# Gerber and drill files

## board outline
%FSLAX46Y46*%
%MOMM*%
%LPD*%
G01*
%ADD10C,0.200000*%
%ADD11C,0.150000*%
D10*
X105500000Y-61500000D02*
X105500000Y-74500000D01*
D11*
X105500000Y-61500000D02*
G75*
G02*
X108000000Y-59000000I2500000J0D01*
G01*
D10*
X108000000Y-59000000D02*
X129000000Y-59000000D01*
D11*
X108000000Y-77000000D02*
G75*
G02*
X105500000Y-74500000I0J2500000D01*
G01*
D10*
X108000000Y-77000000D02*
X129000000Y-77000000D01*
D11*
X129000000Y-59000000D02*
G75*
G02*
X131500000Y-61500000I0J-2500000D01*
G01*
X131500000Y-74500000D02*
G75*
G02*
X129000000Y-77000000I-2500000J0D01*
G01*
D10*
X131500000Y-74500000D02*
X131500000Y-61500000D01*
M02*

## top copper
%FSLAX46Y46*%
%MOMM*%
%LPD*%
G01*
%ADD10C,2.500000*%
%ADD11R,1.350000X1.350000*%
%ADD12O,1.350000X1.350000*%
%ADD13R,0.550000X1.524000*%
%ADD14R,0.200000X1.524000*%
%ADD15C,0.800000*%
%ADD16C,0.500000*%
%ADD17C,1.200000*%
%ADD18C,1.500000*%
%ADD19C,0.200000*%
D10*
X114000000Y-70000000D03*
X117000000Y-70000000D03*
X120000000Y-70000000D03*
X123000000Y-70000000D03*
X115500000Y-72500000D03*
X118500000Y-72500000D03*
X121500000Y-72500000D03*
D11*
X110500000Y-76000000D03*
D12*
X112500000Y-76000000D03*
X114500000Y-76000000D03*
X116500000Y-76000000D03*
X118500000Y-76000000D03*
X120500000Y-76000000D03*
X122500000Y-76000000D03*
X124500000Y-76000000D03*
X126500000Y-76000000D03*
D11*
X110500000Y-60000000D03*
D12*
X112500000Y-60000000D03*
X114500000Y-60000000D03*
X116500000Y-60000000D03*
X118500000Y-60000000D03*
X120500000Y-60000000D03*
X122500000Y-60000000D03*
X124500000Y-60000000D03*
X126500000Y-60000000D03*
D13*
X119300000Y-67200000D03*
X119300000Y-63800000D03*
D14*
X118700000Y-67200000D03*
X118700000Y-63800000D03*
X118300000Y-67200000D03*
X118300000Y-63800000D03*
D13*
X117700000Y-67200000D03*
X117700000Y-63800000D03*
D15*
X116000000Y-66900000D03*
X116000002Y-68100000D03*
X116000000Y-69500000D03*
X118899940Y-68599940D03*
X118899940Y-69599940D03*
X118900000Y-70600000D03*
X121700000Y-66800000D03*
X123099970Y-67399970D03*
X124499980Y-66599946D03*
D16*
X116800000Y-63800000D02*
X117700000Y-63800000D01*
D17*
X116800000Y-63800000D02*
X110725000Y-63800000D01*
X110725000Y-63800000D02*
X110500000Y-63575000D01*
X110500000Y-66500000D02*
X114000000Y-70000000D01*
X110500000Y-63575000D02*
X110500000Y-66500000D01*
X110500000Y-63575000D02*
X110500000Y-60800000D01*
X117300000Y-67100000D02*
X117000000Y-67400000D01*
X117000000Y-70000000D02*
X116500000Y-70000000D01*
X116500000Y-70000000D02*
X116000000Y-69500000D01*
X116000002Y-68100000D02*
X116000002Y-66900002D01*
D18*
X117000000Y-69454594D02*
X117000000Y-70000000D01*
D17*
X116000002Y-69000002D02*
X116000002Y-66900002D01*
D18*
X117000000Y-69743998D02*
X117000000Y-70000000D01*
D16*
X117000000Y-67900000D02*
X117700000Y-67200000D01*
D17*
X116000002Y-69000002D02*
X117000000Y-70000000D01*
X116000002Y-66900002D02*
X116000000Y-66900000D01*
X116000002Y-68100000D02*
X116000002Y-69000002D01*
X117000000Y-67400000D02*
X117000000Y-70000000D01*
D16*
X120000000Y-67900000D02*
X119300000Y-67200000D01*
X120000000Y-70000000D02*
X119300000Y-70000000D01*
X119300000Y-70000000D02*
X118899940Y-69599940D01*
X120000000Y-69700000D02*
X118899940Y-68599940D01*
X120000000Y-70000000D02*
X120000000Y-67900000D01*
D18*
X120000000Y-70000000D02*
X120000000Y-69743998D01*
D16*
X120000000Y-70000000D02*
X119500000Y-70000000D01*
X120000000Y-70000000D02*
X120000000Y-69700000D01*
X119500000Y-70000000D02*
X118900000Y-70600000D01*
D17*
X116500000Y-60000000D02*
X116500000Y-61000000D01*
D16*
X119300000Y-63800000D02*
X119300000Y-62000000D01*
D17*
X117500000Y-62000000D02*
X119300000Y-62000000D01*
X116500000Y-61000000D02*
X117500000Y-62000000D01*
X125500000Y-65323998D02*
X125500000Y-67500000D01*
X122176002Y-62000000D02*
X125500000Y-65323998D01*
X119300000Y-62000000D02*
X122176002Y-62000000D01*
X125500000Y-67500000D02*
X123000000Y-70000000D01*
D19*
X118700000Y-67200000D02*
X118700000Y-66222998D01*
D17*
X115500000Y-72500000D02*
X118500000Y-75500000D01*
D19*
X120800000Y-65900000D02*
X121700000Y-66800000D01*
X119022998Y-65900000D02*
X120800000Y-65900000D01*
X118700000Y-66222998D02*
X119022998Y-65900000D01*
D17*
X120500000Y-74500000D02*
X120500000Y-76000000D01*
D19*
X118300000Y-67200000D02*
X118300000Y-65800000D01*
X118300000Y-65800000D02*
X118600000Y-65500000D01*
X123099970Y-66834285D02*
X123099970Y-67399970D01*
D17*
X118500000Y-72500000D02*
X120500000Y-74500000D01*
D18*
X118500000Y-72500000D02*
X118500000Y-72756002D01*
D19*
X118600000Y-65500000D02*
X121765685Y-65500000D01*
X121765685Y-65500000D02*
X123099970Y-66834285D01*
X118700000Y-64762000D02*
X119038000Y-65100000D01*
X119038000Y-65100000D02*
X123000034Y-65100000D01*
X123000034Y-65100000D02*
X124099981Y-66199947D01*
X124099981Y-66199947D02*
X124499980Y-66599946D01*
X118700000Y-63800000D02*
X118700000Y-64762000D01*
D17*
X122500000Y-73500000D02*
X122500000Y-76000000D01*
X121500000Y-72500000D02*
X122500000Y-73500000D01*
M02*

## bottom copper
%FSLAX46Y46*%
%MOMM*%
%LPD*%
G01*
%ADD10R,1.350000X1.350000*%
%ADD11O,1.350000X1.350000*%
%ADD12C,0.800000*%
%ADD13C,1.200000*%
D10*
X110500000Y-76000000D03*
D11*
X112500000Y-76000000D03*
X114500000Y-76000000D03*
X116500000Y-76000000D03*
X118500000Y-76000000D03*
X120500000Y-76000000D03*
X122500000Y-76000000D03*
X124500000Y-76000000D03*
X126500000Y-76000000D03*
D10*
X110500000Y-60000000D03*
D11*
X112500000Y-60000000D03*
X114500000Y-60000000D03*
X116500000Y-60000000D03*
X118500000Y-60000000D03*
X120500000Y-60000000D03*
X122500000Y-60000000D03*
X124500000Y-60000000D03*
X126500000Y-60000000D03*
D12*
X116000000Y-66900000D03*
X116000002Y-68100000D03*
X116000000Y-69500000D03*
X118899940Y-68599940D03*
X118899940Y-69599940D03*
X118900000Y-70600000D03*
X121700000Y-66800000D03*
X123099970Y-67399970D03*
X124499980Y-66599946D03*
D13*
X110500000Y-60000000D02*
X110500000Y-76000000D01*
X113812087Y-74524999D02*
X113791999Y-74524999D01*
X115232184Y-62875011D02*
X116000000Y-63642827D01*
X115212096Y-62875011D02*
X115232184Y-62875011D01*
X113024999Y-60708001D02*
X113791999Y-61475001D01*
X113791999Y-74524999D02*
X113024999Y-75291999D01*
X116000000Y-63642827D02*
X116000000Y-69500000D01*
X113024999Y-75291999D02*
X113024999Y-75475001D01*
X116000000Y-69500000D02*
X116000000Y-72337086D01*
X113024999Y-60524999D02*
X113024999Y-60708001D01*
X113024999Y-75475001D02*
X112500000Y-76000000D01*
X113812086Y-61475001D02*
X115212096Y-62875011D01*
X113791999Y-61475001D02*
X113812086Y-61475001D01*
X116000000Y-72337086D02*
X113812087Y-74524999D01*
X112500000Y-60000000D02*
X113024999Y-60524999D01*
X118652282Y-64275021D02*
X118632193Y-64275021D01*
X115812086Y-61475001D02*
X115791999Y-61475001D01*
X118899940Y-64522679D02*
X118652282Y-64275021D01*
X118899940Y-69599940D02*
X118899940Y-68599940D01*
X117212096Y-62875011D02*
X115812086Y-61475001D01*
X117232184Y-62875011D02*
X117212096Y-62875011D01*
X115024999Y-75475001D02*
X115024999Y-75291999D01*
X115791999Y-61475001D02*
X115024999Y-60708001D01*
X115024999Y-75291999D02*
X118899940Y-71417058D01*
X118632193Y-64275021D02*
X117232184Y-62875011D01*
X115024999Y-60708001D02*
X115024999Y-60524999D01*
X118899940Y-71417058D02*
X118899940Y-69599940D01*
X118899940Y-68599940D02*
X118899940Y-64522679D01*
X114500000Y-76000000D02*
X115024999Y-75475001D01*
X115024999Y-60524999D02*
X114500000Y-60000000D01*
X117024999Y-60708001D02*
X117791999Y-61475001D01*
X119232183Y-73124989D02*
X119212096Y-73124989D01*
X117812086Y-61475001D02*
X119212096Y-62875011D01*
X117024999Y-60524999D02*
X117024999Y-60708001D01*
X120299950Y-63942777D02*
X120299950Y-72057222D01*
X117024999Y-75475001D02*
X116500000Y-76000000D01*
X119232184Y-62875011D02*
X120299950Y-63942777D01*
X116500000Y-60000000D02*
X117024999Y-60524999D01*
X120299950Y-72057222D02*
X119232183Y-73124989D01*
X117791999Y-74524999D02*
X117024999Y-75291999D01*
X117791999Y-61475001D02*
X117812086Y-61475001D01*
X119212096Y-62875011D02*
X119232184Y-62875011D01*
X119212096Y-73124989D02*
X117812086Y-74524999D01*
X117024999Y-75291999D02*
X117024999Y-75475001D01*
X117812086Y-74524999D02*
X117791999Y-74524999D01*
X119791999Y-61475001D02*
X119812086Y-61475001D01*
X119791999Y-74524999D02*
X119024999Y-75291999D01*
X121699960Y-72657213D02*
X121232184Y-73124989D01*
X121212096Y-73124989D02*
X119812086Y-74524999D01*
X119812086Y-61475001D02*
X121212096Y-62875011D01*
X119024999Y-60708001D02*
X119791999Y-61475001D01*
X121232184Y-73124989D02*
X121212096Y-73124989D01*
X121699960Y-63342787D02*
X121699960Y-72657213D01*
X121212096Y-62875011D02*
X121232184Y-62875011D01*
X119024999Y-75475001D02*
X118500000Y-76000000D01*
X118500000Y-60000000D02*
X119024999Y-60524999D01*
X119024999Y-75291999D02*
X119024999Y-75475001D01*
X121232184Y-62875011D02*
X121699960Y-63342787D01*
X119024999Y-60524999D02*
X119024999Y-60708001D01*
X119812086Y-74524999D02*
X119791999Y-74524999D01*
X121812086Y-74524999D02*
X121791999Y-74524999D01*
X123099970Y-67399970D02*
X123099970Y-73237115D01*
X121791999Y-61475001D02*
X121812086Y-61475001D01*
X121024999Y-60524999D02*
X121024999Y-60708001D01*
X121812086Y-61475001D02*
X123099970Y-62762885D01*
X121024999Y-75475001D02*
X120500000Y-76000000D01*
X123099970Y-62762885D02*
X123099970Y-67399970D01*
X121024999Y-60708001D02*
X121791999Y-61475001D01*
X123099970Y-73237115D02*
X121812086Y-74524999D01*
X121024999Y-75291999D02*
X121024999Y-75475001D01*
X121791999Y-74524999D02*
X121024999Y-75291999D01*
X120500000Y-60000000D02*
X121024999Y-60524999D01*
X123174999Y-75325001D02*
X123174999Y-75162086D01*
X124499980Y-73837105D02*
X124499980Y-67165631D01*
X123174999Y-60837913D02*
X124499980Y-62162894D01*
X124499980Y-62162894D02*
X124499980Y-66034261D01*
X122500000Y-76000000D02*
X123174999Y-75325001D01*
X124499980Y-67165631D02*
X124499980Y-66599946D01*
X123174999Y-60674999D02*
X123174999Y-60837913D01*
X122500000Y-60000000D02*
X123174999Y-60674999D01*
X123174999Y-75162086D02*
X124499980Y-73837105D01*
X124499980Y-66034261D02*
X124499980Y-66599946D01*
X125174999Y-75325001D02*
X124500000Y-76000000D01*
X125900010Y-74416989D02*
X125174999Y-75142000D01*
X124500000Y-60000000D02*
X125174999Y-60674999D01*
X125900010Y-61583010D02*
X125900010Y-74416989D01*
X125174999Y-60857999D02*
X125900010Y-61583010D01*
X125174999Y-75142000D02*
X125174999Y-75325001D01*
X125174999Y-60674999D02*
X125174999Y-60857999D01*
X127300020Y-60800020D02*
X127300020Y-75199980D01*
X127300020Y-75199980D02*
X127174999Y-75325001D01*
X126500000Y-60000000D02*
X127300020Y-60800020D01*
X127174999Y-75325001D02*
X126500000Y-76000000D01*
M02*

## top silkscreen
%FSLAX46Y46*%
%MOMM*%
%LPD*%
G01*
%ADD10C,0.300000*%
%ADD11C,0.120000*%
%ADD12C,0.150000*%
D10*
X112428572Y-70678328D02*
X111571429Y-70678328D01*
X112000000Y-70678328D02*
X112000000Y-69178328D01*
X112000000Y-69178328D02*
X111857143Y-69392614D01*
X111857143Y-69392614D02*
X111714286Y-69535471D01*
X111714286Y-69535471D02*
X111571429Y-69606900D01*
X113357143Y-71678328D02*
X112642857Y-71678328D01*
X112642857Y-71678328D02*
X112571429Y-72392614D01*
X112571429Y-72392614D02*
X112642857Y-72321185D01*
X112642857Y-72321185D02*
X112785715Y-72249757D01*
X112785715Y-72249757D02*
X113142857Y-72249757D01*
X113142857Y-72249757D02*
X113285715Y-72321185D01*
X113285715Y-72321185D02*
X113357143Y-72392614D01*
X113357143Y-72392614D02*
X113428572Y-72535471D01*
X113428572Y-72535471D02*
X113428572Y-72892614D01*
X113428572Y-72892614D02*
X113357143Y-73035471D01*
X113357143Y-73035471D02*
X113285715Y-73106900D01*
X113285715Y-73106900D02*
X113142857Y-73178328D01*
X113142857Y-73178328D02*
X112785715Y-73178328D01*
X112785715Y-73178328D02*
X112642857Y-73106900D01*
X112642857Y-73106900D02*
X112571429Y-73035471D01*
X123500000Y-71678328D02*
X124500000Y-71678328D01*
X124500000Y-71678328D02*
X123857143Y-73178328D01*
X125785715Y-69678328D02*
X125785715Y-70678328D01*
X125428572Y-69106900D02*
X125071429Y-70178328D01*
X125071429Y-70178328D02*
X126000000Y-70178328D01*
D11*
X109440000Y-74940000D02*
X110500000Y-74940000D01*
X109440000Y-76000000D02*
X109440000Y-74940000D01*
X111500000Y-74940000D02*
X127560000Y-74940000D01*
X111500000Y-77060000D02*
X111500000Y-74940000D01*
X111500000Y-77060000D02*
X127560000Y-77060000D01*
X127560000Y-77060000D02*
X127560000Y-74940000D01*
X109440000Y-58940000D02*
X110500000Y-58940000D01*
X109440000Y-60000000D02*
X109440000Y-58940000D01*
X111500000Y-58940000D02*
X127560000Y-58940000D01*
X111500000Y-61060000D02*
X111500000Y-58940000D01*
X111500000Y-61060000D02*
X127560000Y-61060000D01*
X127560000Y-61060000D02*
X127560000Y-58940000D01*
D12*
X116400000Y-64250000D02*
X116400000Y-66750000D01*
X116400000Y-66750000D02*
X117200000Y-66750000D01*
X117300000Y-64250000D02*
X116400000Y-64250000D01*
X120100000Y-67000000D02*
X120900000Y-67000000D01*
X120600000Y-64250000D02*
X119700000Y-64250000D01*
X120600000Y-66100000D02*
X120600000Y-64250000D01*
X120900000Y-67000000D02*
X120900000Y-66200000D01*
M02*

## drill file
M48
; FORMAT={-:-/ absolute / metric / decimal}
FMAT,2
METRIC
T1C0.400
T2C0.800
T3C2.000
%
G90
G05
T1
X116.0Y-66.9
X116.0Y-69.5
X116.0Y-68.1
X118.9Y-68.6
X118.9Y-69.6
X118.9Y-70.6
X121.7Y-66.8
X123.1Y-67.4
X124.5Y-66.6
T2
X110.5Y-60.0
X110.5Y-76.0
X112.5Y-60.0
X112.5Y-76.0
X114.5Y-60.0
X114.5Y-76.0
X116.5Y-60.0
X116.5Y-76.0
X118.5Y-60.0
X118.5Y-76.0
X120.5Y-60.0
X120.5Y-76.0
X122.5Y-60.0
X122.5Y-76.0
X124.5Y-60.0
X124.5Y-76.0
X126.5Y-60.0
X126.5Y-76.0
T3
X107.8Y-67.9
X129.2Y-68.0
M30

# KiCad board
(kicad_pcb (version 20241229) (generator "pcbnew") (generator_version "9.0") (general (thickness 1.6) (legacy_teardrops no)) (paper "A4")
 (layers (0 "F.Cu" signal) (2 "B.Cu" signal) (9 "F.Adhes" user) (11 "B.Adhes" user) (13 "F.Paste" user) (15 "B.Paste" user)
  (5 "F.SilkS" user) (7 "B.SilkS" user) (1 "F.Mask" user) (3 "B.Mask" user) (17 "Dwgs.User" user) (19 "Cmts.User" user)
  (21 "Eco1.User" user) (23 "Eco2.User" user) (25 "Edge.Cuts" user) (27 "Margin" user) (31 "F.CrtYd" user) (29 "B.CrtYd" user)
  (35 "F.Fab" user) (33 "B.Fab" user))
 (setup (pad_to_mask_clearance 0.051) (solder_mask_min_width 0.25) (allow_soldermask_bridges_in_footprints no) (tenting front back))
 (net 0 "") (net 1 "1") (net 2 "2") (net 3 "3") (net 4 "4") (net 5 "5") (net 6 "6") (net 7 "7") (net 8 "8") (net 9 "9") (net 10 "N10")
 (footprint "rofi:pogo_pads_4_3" (layer "F.Cu") (at 118.5 70)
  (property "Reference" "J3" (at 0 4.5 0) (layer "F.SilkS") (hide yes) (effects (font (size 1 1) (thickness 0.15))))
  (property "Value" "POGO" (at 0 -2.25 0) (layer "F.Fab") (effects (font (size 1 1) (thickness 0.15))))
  (pad "1" smd circle (at -4.5 0) (size 2.5 2.5) (layers "F.Cu" "F.Mask" "F.Paste") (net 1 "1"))
  (pad "2" smd circle (at -1.5 0) (size 2.5 2.5) (layers "F.Cu" "F.Mask" "F.Paste") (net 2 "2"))
  (pad "3" smd circle (at 1.5 0) (size 2.5 2.5) (layers "F.Cu" "F.Mask" "F.Paste") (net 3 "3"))
  (pad "4" smd circle (at 4.5 0) (size 2.5 2.5) (layers "F.Cu" "F.Mask" "F.Paste") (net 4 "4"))
  (pad "5" smd circle (at -3 2.5) (size 2.5 2.5) (layers "F.Cu" "F.Mask" "F.Paste") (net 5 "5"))
  (pad "6" smd circle (at 0 2.5) (size 2.5 2.5) (layers "F.Cu" "F.Mask" "F.Paste") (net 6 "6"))
  (pad "7" smd circle (at 3 2.5) (size 2.5 2.5) (layers "F.Cu" "F.Mask" "F.Paste") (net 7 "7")))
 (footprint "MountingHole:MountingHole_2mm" (layer "F.Cu") (at 129.2 68)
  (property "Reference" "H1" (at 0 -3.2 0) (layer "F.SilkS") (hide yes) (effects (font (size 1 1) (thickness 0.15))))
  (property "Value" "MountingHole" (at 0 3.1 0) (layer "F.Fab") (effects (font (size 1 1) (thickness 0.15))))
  (pad "" np_thru_hole circle (at 0 0) (size 2 2) (drill 2) (layers "*.Cu" "*.Mask")))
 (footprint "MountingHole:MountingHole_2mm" (layer "F.Cu") (at 107.8 67.9)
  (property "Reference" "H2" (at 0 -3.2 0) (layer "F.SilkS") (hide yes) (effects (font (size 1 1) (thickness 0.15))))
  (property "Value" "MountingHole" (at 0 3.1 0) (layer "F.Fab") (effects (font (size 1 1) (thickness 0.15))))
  (pad "" np_thru_hole circle (at 0 0) (size 2 2) (drill 2) (layers "*.Cu" "*.Mask")))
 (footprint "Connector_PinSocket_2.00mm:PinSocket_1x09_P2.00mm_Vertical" (layer "F.Cu") (at 110.5 76 90)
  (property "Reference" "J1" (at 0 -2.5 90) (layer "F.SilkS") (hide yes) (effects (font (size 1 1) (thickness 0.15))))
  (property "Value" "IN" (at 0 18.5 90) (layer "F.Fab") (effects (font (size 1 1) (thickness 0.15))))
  (fp_line (start 1.06 -1.06) (end 1.06 0) (stroke (width 0.12) (type solid)) (layer "F.SilkS"))
  (fp_line (start 0 -1.06) (end 1.06 -1.06) (stroke (width 0.12) (type solid)) (layer "F.SilkS"))
  (fp_line (start 1.06 1) (end 1.06 17.06) (stroke (width 0.12) (type solid)) (layer "F.SilkS"))
  (fp_line (start -1.06 1) (end 1.06 1) (stroke (width 0.12) (type solid)) (layer "F.SilkS"))
  (fp_line (start -1.06 1) (end -1.06 17.06) (stroke (width 0.12) (type solid)) (layer "F.SilkS"))
  (fp_line (start -1.06 17.06) (end 1.06 17.06) (stroke (width 0.12) (type solid)) (layer "F.SilkS"))
  (pad "1" thru_hole rect (at 0 0 90) (size 1.35 1.35) (drill 0.8) (layers "*.Cu" "*.Mask") (remove_unused_layers no) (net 1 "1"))
  (pad "2" thru_hole oval (at 0 2 90) (size 1.35 1.35) (drill 0.8) (layers "*.Cu" "*.Mask") (remove_unused_layers no) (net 2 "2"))
  (pad "3" thru_hole oval (at 0 4 90) (size 1.35 1.35) (drill 0.8) (layers "*.Cu" "*.Mask") (remove_unused_layers no) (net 3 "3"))
  (pad "4" thru_hole oval (at 0 6 90) (size 1.35 1.35) (drill 0.8) (layers "*.Cu" "*.Mask") (remove_unused_layers no) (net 4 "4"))
  (pad "5" thru_hole oval (at 0 8 90) (size 1.35 1.35) (drill 0.8) (layers "*.Cu" "*.Mask") (remove_unused_layers no) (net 5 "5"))
  (pad "6" thru_hole oval (at 0 10 90) (size 1.35 1.35) (drill 0.8) (layers "*.Cu" "*.Mask") (remove_unused_layers no) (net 6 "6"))
  (pad "7" thru_hole oval (at 0 12 90) (size 1.35 1.35) (drill 0.8) (layers "*.Cu" "*.Mask") (remove_unused_layers no) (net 7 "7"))
  (pad "8" thru_hole oval (at 0 14 90) (size 1.35 1.35) (drill 0.8) (layers "*.Cu" "*.Mask") (remove_unused_layers no) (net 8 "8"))
  (pad "9" thru_hole oval (at 0 16 90) (size 1.35 1.35) (drill 0.8) (layers "*.Cu" "*.Mask") (remove_unused_layers no) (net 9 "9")))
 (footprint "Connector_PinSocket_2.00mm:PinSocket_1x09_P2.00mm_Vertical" (layer "F.Cu") (at 110.5 60 90)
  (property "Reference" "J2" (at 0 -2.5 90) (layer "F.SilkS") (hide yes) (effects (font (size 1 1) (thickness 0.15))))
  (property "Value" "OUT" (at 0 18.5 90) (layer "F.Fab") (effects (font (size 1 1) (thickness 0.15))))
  (fp_line (start 1.06 -1.06) (end 1.06 0) (stroke (width 0.12) (type solid)) (layer "F.SilkS"))
  (fp_line (start 0 -1.06) (end 1.06 -1.06) (stroke (width 0.12) (type solid)) (layer "F.SilkS"))
  (fp_line (start 1.06 1) (end 1.06 17.06) (stroke (width 0.12) (type solid)) (layer "F.SilkS"))
  (fp_line (start -1.06 1) (end 1.06 1) (stroke (width 0.12) (type solid)) (layer "F.SilkS"))
  (fp_line (start -1.06 1) (end -1.06 17.06) (stroke (width 0.12) (type solid)) (layer "F.SilkS"))
  (fp_line (start -1.06 17.06) (end 1.06 17.06) (stroke (width 0.12) (type solid)) (layer "F.SilkS"))
  (pad "1" thru_hole rect (at 0 0 90) (size 1.35 1.35) (drill 0.8) (layers "*.Cu" "*.Mask") (remove_unused_layers no) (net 1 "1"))
  (pad "2" thru_hole oval (at 0 2 90) (size 1.35 1.35) (drill 0.8) (layers "*.Cu" "*.Mask") (remove_unused_layers no) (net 2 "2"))
  (pad "3" thru_hole oval (at 0 4 90) (size 1.35 1.35) (drill 0.8) (layers "*.Cu" "*.Mask") (remove_unused_layers no) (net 3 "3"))
  (pad "4" thru_hole oval (at 0 6 90) (size 1.35 1.35) (drill 0.8) (layers "*.Cu" "*.Mask") (remove_unused_layers no) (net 4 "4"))
  (pad "5" thru_hole oval (at 0 8 90) (size 1.35 1.35) (drill 0.8) (layers "*.Cu" "*.Mask") (remove_unused_layers no) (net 5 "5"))
  (pad "6" thru_hole oval (at 0 10 90) (size 1.35 1.35) (drill 0.8) (layers "*.Cu" "*.Mask") (remove_unused_layers no) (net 6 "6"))
  (pad "7" thru_hole oval (at 0 12 90) (size 1.35 1.35) (drill 0.8) (layers "*.Cu" "*.Mask") (remove_unused_layers no) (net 7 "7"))
  (pad "8" thru_hole oval (at 0 14 90) (size 1.35 1.35) (drill 0.8) (layers "*.Cu" "*.Mask") (remove_unused_layers no) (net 8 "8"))
  (pad "9" thru_hole oval (at 0 16 90) (size 1.35 1.35) (drill 0.8) (layers "*.Cu" "*.Mask") (remove_unused_layers no) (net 9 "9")))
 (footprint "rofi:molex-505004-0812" (layer "F.Cu") (at 118.5 65.5 180)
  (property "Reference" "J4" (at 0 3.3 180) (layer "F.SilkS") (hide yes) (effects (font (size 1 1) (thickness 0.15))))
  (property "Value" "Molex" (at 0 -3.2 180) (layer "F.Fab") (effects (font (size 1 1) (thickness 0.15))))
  (fp_line (start 2.1 1.25) (end 2.1 -1.25) (stroke (width 0.15) (type solid)) (layer "F.SilkS"))
  (fp_line (start 2.1 -1.25) (end 1.3 -1.25) (stroke (width 0.15) (type solid)) (layer "F.SilkS"))
  (fp_line (start 1.2 1.25) (end 2.1 1.25) (stroke (width 0.15) (type solid)) (layer "F.SilkS"))
  (fp_line (start -1.6 -1.5) (end -2.4 -1.5) (stroke (width 0.15) (type solid)) (layer "F.SilkS"))
  (fp_line (start -2.1 1.25) (end -1.2 1.25) (stroke (width 0.15) (type solid)) (layer "F.SilkS"))
  (fp_line (start -2.1 -0.6) (end -2.1 1.25) (stroke (width 0.15) (type solid)) (layer "F.SilkS"))
  (fp_line (start -2.4 -1.5) (end -2.4 -0.7) (stroke (width 0.15) (type solid)) (layer "F.SilkS"))
  (pad "1" smd rect (at -0.8 -1.7 180) (size 0.55 1.524) (layers "F.Cu" "F.Mask" "F.Paste") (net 3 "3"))
  (pad "2" smd rect (at -0.8 1.7 180) (size 0.55 1.524) (layers "F.Cu" "F.Mask" "F.Paste") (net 4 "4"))
  (pad "3" smd rect (at -0.2 -1.7 180) (size 0.2 1.524) (layers "F.Cu" "F.Mask" "F.Paste") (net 5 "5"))
  (pad "4" smd rect (at -0.2 1.7 180) (size 0.2 1.524) (layers "F.Cu" "F.Mask" "F.Paste") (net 7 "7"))
  (pad "5" smd rect (at 0.2 -1.7 180) (size 0.2 1.524) (layers "F.Cu" "F.Mask" "F.Paste") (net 6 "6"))
  (pad "6" smd rect (at 0.2 1.7 180) (size 0.2 1.524) (layers "F.Cu" "F.Mask" "F.Paste") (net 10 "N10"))
  (pad "7" smd rect (at 0.8 -1.7 180) (size 0.55 1.524) (layers "F.Cu" "F.Mask" "F.Paste") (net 2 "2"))
  (pad "8" smd rect (at 0.8 1.7 180) (size 0.55 1.524) (layers "F.Cu" "F.Mask" "F.Paste") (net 1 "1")))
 (gr_line (start 105.5 61.5) (end 105.5 74.5) (stroke (width 0.2) (type solid)) (layer "Edge.Cuts"))
 (gr_arc (start 105.5 61.5) (mid 106.232233 59.732233) (end 108 59) (stroke (width 0.15) (type solid)) (layer "Edge.Cuts"))
 (gr_line (start 108 59) (end 129 59) (stroke (width 0.2) (type solid)) (layer "Edge.Cuts"))
 (gr_arc (start 108 77) (mid 106.232233 76.267767) (end 105.5 74.5) (stroke (width 0.15) (type solid)) (layer "Edge.Cuts"))
 (gr_line (start 108 77) (end 129 77) (stroke (width 0.2) (type solid)) (layer "Edge.Cuts"))
 (gr_arc (start 129 59) (mid 130.767767 59.732233) (end 131.5 61.5) (stroke (width 0.15) (type solid)) (layer "Edge.Cuts"))
 (gr_arc (start 131.5 74.5) (mid 130.767767 76.267767) (end 129 77) (stroke (width 0.15) (type solid)) (layer "Edge.Cuts"))
 (gr_line (start 131.5 74.5) (end 131.5 61.5) (stroke (width 0.2) (type solid)) (layer "Edge.Cuts"))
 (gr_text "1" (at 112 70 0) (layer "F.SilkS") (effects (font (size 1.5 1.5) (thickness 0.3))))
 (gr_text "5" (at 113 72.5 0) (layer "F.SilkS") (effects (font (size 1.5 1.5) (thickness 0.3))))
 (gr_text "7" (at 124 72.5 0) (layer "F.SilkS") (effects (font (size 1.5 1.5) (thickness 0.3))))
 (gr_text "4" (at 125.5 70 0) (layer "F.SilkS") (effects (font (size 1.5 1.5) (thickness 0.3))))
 (segment (start 116.8 63.8) (end 117.7 63.8) (width 0.5) (layer "F.Cu") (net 1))
 (segment (start 116.8 63.8) (end 110.725 63.8) (width 1.2) (layer "F.Cu") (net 1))
 (segment (start 110.725 63.8) (end 110.5 63.575) (width 1.2) (layer "F.Cu") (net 1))
 (segment (start 110.5 66.5) (end 114 70) (width 1.2) (layer "F.Cu") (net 1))
 (segment (start 110.5 63.575) (end 110.5 66.5) (width 1.2) (layer "F.Cu") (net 1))
 (segment (start 110.5 63.575) (end 110.5 60.8) (width 1.2) (layer "F.Cu") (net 1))
 (segment (start 110.5 60) (end 110.5 76) (width 1.2) (layer "B.Cu") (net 1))
 (segment (start 117.3 67.1) (end 117 67.4) (width 1.2) (layer "F.Cu") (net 2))
 (segment (start 117 70) (end 116.5 70) (width 1.2) (layer "F.Cu") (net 2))
 (segment (start 116.5 70) (end 116 69.5) (width 1.2) (layer "F.Cu") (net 2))
 (segment (start 116.000002 68.1) (end 116.000002 66.900002) (width 1.2) (layer "F.Cu") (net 2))
 (segment (start 117 69.454594) (end 117 70) (width 1.5) (layer "F.Cu") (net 2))
 (segment (start 116.000002 69.000002) (end 116.000002 66.900002) (width 1.2) (layer "F.Cu") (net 2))
 (segment (start 117 69.743998) (end 117 70) (width 1.5) (layer "F.Cu") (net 2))
 (segment (start 117 67.9) (end 117.7 67.2) (width 0.5) (layer "F.Cu") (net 2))
 (segment (start 116.000002 69.000002) (end 117 70) (width 1.2) (layer "F.Cu") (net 2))
 (segment (start 116.000002 66.900002) (end 116 66.9) (width 1.2) (layer "F.Cu") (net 2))
 (segment (start 116.000002 68.1) (end 116.000002 69.000002) (width 1.2) (layer "F.Cu") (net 2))
 (segment (start 117 67.4) (end 117 70) (width 1.2) (layer "F.Cu") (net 2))
 (via (at 116 66.9) (size 0.8) (drill 0.4) (layers "F.Cu" "B.Cu") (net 2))
 (via (at 116.000002 68.1) (size 0.8) (drill 0.4) (layers "F.Cu" "B.Cu") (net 2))
 (via (at 116 69.5) (size 0.8) (drill 0.4) (layers "F.Cu" "B.Cu") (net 2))
 (segment (start 113.812087 74.524999) (end 113.791999 74.524999) (width 1.2) (layer "B.Cu") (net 2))
 (segment (start 115.232184 62.875011) (end 116 63.642827) (width 1.2) (layer "B.Cu") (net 2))
 (segment (start 115.212096 62.875011) (end 115.232184 62.875011) (width 1.2) (layer "B.Cu") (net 2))
 (segment (start 113.024999 60.708001) (end 113.791999 61.475001) (width 1.2) (layer "B.Cu") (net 2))
 (segment (start 113.791999 74.524999) (end 113.024999 75.291999) (width 1.2) (layer "B.Cu") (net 2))
 (segment (start 116 63.642827) (end 116 69.5) (width 1.2) (layer "B.Cu") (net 2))
 (segment (start 113.024999 75.291999) (end 113.024999 75.475001) (width 1.2) (layer "B.Cu") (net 2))
 (segment (start 116 69.5) (end 116 72.337086) (width 1.2) (layer "B.Cu") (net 2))
 (segment (start 113.024999 60.524999) (end 113.024999 60.708001) (width 1.2) (layer "B.Cu") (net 2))
 (segment (start 113.024999 75.475001) (end 112.5 76) (width 1.2) (layer "B.Cu") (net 2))
 (segment (start 113.812086 61.475001) (end 115.212096 62.875011) (width 1.2) (layer "B.Cu") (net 2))
 (segment (start 113.791999 61.475001) (end 113.812086 61.475001) (width 1.2) (layer "B.Cu") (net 2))
 (segment (start 116 72.337086) (end 113.812087 74.524999) (width 1.2) (layer "B.Cu") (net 2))
 (segment (start 112.5 60) (end 113.024999 60.524999) (width 1.2) (layer "B.Cu") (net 2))
 (segment (start 120 67.9) (end 119.3 67.2) (width 0.5) (layer "F.Cu") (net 3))
 (segment (start 120 70) (end 119.3 70) (width 0.5) (layer "F.Cu") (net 3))
 (segment (start 119.3 70) (end 118.89994 69.59994) (width 0.5) (layer "F.Cu") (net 3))
 (segment (start 120 69.7) (end 118.89994 68.59994) (width 0.5) (layer "F.Cu") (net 3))
 (segment (start 120 70) (end 120 67.9) (width 0.5) (layer "F.Cu") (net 3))
 (segment (start 120 70) (end 120 69.743998) (width 1.5) (layer "F.Cu") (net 3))
 (segment (start 120 70) (end 119.5 70) (width 0.5) (layer "F.Cu") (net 3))
 (segment (start 120 70) (end 120 69.7) (width 0.5) (layer "F.Cu") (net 3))
 (segment (start 119.5 70) (end 118.9 70.6) (width 0.5) (layer "F.Cu") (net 3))
 (via (at 118.89994 68.59994) (size 0.8) (drill 0.4) (layers "F.Cu" "B.Cu") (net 3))
 (via (at 118.89994 69.59994) (size 0.8) (drill 0.4) (layers "F.Cu" "B.Cu") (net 3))
 (via (at 118.9 70.6) (size 0.8) (drill 0.4) (layers "F.Cu" "B.Cu") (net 3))
 (segment (start 118.652282 64.275021) (end 118.632193 64.275021) (width 1.2) (layer "B.Cu") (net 3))
 (segment (start 115.812086 61.475001) (end 115.791999 61.475001) (width 1.2) (layer "B.Cu") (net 3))
 (segment (start 118.89994 64.522679) (end 118.652282 64.275021) (width 1.2) (layer "B.Cu") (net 3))
 (segment (start 118.89994 69.59994) (end 118.89994 68.59994) (width 1.2) (layer "B.Cu") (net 3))
 (segment (start 117.212096 62.875011) (end 115.812086 61.475001) (width 1.2) (layer "B.Cu") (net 3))
 (segment (start 117.232184 62.875011) (end 117.212096 62.875011) (width 1.2) (layer "B.Cu") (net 3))
 (segment (start 115.024999 75.475001) (end 115.024999 75.291999) (width 1.2) (layer "B.Cu") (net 3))
 (segment (start 115.791999 61.475001) (end 115.024999 60.708001) (width 1.2) (layer "B.Cu") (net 3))
 (segment (start 115.024999 75.291999) (end 118.89994 71.417058) (width 1.2) (layer "B.Cu") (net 3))
 (segment (start 118.632193 64.275021) (end 117.232184 62.875011) (width 1.2) (layer "B.Cu") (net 3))
 (segment (start 115.024999 60.708001) (end 115.024999 60.524999) (width 1.2) (layer "B.Cu") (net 3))
 (segment (start 118.89994 71.417058) (end 118.89994 69.59994) (width 1.2) (layer "B.Cu") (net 3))
 (segment (start 118.89994 68.59994) (end 118.89994 64.522679) (width 1.2) (layer "B.Cu") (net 3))
 (segment (start 114.5 76) (end 115.024999 75.475001) (width 1.2) (layer "B.Cu") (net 3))
 (segment (start 115.024999 60.524999) (end 114.5 60) (width 1.2) (layer "B.Cu") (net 3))
 (segment (start 116.5 60) (end 116.5 61) (width 1.2) (layer "F.Cu") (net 4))
 (segment (start 119.3 63.8) (end 119.3 62) (width 0.5) (layer "F.Cu") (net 4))
 (segment (start 117.5 62) (end 119.3 62) (width 1.2) (layer "F.Cu") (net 4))
 (segment (start 116.5 61) (end 117.5 62) (width 1.2) (layer "F.Cu") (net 4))
 (segment (start 125.5 65.323998) (end 125.5 67.5) (width 1.2) (layer "F.Cu") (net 4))
 (segment (start 122.176002 62) (end 125.5 65.323998) (width 1.2) (layer "F.Cu") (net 4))
 (segment (start 119.3 62) (end 122.176002 62) (width 1.2) (layer "F.Cu") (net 4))
 (segment (start 125.5 67.5) (end 123 70) (width 1.2) (layer "F.Cu") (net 4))
 (segment (start 117.024999 60.708001) (end 117.791999 61.475001) (width 1.2) (layer "B.Cu") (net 4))
 (segment (start 119.232183 73.124989) (end 119.212096 73.124989) (width 1.2) (layer "B.Cu") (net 4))
 (segment (start 117.812086 61.475001) (end 119.212096 62.875011) (width 1.2) (layer "B.Cu") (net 4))
 (segment (start 117.024999 60.524999) (end 117.024999 60.708001) (width 1.2) (layer "B.Cu") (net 4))
 (segment (start 120.29995 63.942777) (end 120.29995 72.057222) (width 1.2) (layer "B.Cu") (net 4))
 (segment (start 117.024999 75.475001) (end 116.5 76) (width 1.2) (layer "B.Cu") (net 4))
 (segment (start 119.232184 62.875011) (end 120.29995 63.942777) (width 1.2) (layer "B.Cu") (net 4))
 (segment (start 116.5 60) (end 117.024999 60.524999) (width 1.2) (layer "B.Cu") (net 4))
 (segment (start 120.29995 72.057222) (end 119.232183 73.124989) (width 1.2) (layer "B.Cu") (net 4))
 (segment (start 117.791999 74.524999) (end 117.024999 75.291999) (width 1.2) (layer "B.Cu") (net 4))
 (segment (start 117.791999 61.475001) (end 117.812086 61.475001) (width 1.2) (layer "B.Cu") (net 4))
 (segment (start 119.212096 62.875011) (end 119.232184 62.875011) (width 1.2) (layer "B.Cu") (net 4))
 (segment (start 119.212096 73.124989) (end 117.812086 74.524999) (width 1.2) (layer "B.Cu") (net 4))
 (segment (start 117.024999 75.291999) (end 117.024999 75.475001) (width 1.2) (layer "B.Cu") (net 4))
 (segment (start 117.812086 74.524999) (end 117.791999 74.524999) (width 1.2) (layer "B.Cu") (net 4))
 (segment (start 118.7 67.2) (end 118.7 66.222998) (width 0.2) (layer "F.Cu") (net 5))
 (segment (start 115.5 72.5) (end 118.5 75.5) (width 1.2) (layer "F.Cu") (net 5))
 (segment (start 120.8 65.9) (end 121.7 66.8) (width 0.2) (layer "F.Cu") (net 5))
 (segment (start 119.022998 65.9) (end 120.8 65.9) (width 0.2) (layer "F.Cu") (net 5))
 (segment (start 118.7 66.222998) (end 119.022998 65.9) (width 0.2) (layer "F.Cu") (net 5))
 (via (at 121.7 66.8) (size 0.8) (drill 0.4) (layers "F.Cu" "B.Cu") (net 5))
 (segment (start 119.791999 61.475001) (end 119.812086 61.475001) (width 1.2) (layer "B.Cu") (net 5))
 (segment (start 119.791999 74.524999) (end 119.024999 75.291999) (width 1.2) (layer "B.Cu") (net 5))
 (segment (start 121.69996 72.657213) (end 121.232184 73.124989) (width 1.2) (layer "B.Cu") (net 5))
 (segment (start 121.212096 73.124989) (end 119.812086 74.524999) (width 1.2) (layer "B.Cu") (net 5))
 (segment (start 119.812086 61.475001) (end 121.212096 62.875011) (width 1.2) (layer "B.Cu") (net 5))
 (segment (start 119.024999 60.708001) (end 119.791999 61.475001) (width 1.2) (layer "B.Cu") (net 5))
 (segment (start 121.232184 73.124989) (end 121.212096 73.124989) (width 1.2) (layer "B.Cu") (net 5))
 (segment (start 121.69996 63.342787) (end 121.69996 72.657213) (width 1.2) (layer "B.Cu") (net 5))
 (segment (start 121.212096 62.875011) (end 121.232184 62.875011) (width 1.2) (layer "B.Cu") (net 5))
 (segment (start 119.024999 75.475001) (end 118.5 76) (width 1.2) (layer "B.Cu") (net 5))
 (segment (start 118.5 60) (end 119.024999 60.524999) (width 1.2) (layer "B.Cu") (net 5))
 (segment (start 119.024999 75.291999) (end 119.024999 75.475001) (width 1.2) (layer "B.Cu") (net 5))
 (segment (start 121.232184 62.875011) (end 121.69996 63.342787) (width 1.2) (layer "B.Cu") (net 5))
 (segment (start 119.024999 60.524999) (end 119.024999 60.708001) (width 1.2) (layer "B.Cu") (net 5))
 (segment (start 119.812086 74.524999) (end 119.791999 74.524999) (width 1.2) (layer "B.Cu") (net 5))
 (segment (start 120.5 74.5) (end 120.5 76) (width 1.2) (layer "F.Cu") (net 6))
 (segment (start 118.3 67.2) (end 118.3 65.8) (width 0.2) (layer "F.Cu") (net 6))
 (segment (start 118.3 65.8) (end 118.6 65.5) (width 0.2) (layer "F.Cu") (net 6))
 (segment (start 123.09997 66.834285) (end 123.09997 67.39997) (width 0.2) (layer "F.Cu") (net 6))
 (segment (start 118.5 72.5) (end 120.5 74.5) (width 1.2) (layer "F.Cu") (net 6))
 (segment (start 118.5 72.5) (end 118.5 72.756002) (width 1.5) (layer "F.Cu") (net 6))
 (segment (start 118.6 65.5) (end 121.765685 65.5) (width 0.2) (layer "F.Cu") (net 6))
 (segment (start 121.765685 65.5) (end 123.09997 66.834285) (width 0.2) (layer "F.Cu") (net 6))
 (via (at 123.09997 67.39997) (size 0.8) (drill 0.4) (layers "F.Cu" "B.Cu") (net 6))
 (segment (start 121.812086 74.524999) (end 121.791999 74.524999) (width 1.2) (layer "B.Cu") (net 6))
 (segment (start 123.09997 67.39997) (end 123.09997 73.237115) (width 1.2) (layer "B.Cu") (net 6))
 (segment (start 121.791999 61.475001) (end 121.812086 61.475001) (width 1.2) (layer "B.Cu") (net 6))
 (segment (start 121.024999 60.524999) (end 121.024999 60.708001) (width 1.2) (layer "B.Cu") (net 6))
 (segment (start 121.812086 61.475001) (end 123.09997 62.762885) (width 1.2) (layer "B.Cu") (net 6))
 (segment (start 121.024999 75.475001) (end 120.5 76) (width 1.2) (layer "B.Cu") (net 6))
 (segment (start 123.09997 62.762885) (end 123.09997 67.39997) (width 1.2) (layer "B.Cu") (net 6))
 (segment (start 121.024999 60.708001) (end 121.791999 61.475001) (width 1.2) (layer "B.Cu") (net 6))
 (segment (start 123.09997 73.237115) (end 121.812086 74.524999) (width 1.2) (layer "B.Cu") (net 6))
 (segment (start 121.024999 75.291999) (end 121.024999 75.475001) (width 1.2) (layer "B.Cu") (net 6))
 (segment (start 121.791999 74.524999) (end 121.024999 75.291999) (width 1.2) (layer "B.Cu") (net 6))
 (segment (start 120.5 60) (end 121.024999 60.524999) (width 1.2) (layer "B.Cu") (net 6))
 (segment (start 118.7 64.762) (end 119.038 65.1) (width 0.2) (layer "F.Cu") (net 7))
 (segment (start 119.038 65.1) (end 123.000034 65.1) (width 0.2) (layer "F.Cu") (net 7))
 (segment (start 123.000034 65.1) (end 124.099981 66.199947) (width 0.2) (layer "F.Cu") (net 7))
 (segment (start 124.099981 66.199947) (end 124.49998 66.599946) (width 0.2) (layer "F.Cu") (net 7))
 (segment (start 118.7 63.8) (end 118.7 64.762) (width 0.2) (layer "F.Cu") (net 7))
 (segment (start 122.5 73.5) (end 122.5 76) (width 1.2) (layer "F.Cu") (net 7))
 (segment (start 121.5 72.5) (end 122.5 73.5) (width 1.2) (layer "F.Cu") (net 7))
 (via (at 124.49998 66.599946) (size 0.8) (drill 0.4) (layers "F.Cu" "B.Cu") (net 7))
 (segment (start 123.174999 75.325001) (end 123.174999 75.162086) (width 1.2) (layer "B.Cu") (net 7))
 (segment (start 124.49998 73.837105) (end 124.49998 67.165631) (width 1.2) (layer "B.Cu") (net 7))
 (segment (start 123.174999 60.837913) (end 124.49998 62.162894) (width 1.2) (layer "B.Cu") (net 7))
 (segment (start 124.49998 62.162894) (end 124.49998 66.034261) (width 1.2) (layer "B.Cu") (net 7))
 (segment (start 122.5 76) (end 123.174999 75.325001) (width 1.2) (layer "B.Cu") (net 7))
 (segment (start 124.49998 67.165631) (end 124.49998 66.599946) (width 1.2) (layer "B.Cu") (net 7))
 (segment (start 123.174999 60.674999) (end 123.174999 60.837913) (width 1.2) (layer "B.Cu") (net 7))
 (segment (start 122.5 60) (end 123.174999 60.674999) (width 1.2) (layer "B.Cu") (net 7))
 (segment (start 123.174999 75.162086) (end 124.49998 73.837105) (width 1.2) (layer "B.Cu") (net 7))
 (segment (start 124.49998 66.034261) (end 124.49998 66.599946) (width 1.2) (layer "B.Cu") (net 7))
 (segment (start 125.174999 75.325001) (end 124.5 76) (width 1.2) (layer "B.Cu") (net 8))
 (segment (start 125.90001 74.416989) (end 125.174999 75.142) (width 1.2) (layer "B.Cu") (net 8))
 (segment (start 124.5 60) (end 125.174999 60.674999) (width 1.2) (layer "B.Cu") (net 8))
 (segment (start 125.90001 61.58301) (end 125.90001 74.416989) (width 1.2) (layer "B.Cu") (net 8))
 (segment (start 125.174999 60.857999) (end 125.90001 61.58301) (width 1.2) (layer "B.Cu") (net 8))
 (segment (start 125.174999 75.142) (end 125.174999 75.325001) (width 1.2) (layer "B.Cu") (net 8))
 (segment (start 125.174999 60.674999) (end 125.174999 60.857999) (width 1.2) (layer "B.Cu") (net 8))
 (segment (start 127.30002 60.80002) (end 127.30002 75.19998) (width 1.2) (layer "B.Cu") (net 9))
 (segment (start 127.30002 75.19998) (end 127.174999 75.325001) (width 1.2) (layer "B.Cu") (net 9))
 (segment (start 126.5 60) (end 127.30002 60.80002) (width 1.2) (layer "B.Cu") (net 9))
 (segment (start 127.174999 75.325001) (end 126.5 76) (width 1.2) (layer "B.Cu") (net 9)))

